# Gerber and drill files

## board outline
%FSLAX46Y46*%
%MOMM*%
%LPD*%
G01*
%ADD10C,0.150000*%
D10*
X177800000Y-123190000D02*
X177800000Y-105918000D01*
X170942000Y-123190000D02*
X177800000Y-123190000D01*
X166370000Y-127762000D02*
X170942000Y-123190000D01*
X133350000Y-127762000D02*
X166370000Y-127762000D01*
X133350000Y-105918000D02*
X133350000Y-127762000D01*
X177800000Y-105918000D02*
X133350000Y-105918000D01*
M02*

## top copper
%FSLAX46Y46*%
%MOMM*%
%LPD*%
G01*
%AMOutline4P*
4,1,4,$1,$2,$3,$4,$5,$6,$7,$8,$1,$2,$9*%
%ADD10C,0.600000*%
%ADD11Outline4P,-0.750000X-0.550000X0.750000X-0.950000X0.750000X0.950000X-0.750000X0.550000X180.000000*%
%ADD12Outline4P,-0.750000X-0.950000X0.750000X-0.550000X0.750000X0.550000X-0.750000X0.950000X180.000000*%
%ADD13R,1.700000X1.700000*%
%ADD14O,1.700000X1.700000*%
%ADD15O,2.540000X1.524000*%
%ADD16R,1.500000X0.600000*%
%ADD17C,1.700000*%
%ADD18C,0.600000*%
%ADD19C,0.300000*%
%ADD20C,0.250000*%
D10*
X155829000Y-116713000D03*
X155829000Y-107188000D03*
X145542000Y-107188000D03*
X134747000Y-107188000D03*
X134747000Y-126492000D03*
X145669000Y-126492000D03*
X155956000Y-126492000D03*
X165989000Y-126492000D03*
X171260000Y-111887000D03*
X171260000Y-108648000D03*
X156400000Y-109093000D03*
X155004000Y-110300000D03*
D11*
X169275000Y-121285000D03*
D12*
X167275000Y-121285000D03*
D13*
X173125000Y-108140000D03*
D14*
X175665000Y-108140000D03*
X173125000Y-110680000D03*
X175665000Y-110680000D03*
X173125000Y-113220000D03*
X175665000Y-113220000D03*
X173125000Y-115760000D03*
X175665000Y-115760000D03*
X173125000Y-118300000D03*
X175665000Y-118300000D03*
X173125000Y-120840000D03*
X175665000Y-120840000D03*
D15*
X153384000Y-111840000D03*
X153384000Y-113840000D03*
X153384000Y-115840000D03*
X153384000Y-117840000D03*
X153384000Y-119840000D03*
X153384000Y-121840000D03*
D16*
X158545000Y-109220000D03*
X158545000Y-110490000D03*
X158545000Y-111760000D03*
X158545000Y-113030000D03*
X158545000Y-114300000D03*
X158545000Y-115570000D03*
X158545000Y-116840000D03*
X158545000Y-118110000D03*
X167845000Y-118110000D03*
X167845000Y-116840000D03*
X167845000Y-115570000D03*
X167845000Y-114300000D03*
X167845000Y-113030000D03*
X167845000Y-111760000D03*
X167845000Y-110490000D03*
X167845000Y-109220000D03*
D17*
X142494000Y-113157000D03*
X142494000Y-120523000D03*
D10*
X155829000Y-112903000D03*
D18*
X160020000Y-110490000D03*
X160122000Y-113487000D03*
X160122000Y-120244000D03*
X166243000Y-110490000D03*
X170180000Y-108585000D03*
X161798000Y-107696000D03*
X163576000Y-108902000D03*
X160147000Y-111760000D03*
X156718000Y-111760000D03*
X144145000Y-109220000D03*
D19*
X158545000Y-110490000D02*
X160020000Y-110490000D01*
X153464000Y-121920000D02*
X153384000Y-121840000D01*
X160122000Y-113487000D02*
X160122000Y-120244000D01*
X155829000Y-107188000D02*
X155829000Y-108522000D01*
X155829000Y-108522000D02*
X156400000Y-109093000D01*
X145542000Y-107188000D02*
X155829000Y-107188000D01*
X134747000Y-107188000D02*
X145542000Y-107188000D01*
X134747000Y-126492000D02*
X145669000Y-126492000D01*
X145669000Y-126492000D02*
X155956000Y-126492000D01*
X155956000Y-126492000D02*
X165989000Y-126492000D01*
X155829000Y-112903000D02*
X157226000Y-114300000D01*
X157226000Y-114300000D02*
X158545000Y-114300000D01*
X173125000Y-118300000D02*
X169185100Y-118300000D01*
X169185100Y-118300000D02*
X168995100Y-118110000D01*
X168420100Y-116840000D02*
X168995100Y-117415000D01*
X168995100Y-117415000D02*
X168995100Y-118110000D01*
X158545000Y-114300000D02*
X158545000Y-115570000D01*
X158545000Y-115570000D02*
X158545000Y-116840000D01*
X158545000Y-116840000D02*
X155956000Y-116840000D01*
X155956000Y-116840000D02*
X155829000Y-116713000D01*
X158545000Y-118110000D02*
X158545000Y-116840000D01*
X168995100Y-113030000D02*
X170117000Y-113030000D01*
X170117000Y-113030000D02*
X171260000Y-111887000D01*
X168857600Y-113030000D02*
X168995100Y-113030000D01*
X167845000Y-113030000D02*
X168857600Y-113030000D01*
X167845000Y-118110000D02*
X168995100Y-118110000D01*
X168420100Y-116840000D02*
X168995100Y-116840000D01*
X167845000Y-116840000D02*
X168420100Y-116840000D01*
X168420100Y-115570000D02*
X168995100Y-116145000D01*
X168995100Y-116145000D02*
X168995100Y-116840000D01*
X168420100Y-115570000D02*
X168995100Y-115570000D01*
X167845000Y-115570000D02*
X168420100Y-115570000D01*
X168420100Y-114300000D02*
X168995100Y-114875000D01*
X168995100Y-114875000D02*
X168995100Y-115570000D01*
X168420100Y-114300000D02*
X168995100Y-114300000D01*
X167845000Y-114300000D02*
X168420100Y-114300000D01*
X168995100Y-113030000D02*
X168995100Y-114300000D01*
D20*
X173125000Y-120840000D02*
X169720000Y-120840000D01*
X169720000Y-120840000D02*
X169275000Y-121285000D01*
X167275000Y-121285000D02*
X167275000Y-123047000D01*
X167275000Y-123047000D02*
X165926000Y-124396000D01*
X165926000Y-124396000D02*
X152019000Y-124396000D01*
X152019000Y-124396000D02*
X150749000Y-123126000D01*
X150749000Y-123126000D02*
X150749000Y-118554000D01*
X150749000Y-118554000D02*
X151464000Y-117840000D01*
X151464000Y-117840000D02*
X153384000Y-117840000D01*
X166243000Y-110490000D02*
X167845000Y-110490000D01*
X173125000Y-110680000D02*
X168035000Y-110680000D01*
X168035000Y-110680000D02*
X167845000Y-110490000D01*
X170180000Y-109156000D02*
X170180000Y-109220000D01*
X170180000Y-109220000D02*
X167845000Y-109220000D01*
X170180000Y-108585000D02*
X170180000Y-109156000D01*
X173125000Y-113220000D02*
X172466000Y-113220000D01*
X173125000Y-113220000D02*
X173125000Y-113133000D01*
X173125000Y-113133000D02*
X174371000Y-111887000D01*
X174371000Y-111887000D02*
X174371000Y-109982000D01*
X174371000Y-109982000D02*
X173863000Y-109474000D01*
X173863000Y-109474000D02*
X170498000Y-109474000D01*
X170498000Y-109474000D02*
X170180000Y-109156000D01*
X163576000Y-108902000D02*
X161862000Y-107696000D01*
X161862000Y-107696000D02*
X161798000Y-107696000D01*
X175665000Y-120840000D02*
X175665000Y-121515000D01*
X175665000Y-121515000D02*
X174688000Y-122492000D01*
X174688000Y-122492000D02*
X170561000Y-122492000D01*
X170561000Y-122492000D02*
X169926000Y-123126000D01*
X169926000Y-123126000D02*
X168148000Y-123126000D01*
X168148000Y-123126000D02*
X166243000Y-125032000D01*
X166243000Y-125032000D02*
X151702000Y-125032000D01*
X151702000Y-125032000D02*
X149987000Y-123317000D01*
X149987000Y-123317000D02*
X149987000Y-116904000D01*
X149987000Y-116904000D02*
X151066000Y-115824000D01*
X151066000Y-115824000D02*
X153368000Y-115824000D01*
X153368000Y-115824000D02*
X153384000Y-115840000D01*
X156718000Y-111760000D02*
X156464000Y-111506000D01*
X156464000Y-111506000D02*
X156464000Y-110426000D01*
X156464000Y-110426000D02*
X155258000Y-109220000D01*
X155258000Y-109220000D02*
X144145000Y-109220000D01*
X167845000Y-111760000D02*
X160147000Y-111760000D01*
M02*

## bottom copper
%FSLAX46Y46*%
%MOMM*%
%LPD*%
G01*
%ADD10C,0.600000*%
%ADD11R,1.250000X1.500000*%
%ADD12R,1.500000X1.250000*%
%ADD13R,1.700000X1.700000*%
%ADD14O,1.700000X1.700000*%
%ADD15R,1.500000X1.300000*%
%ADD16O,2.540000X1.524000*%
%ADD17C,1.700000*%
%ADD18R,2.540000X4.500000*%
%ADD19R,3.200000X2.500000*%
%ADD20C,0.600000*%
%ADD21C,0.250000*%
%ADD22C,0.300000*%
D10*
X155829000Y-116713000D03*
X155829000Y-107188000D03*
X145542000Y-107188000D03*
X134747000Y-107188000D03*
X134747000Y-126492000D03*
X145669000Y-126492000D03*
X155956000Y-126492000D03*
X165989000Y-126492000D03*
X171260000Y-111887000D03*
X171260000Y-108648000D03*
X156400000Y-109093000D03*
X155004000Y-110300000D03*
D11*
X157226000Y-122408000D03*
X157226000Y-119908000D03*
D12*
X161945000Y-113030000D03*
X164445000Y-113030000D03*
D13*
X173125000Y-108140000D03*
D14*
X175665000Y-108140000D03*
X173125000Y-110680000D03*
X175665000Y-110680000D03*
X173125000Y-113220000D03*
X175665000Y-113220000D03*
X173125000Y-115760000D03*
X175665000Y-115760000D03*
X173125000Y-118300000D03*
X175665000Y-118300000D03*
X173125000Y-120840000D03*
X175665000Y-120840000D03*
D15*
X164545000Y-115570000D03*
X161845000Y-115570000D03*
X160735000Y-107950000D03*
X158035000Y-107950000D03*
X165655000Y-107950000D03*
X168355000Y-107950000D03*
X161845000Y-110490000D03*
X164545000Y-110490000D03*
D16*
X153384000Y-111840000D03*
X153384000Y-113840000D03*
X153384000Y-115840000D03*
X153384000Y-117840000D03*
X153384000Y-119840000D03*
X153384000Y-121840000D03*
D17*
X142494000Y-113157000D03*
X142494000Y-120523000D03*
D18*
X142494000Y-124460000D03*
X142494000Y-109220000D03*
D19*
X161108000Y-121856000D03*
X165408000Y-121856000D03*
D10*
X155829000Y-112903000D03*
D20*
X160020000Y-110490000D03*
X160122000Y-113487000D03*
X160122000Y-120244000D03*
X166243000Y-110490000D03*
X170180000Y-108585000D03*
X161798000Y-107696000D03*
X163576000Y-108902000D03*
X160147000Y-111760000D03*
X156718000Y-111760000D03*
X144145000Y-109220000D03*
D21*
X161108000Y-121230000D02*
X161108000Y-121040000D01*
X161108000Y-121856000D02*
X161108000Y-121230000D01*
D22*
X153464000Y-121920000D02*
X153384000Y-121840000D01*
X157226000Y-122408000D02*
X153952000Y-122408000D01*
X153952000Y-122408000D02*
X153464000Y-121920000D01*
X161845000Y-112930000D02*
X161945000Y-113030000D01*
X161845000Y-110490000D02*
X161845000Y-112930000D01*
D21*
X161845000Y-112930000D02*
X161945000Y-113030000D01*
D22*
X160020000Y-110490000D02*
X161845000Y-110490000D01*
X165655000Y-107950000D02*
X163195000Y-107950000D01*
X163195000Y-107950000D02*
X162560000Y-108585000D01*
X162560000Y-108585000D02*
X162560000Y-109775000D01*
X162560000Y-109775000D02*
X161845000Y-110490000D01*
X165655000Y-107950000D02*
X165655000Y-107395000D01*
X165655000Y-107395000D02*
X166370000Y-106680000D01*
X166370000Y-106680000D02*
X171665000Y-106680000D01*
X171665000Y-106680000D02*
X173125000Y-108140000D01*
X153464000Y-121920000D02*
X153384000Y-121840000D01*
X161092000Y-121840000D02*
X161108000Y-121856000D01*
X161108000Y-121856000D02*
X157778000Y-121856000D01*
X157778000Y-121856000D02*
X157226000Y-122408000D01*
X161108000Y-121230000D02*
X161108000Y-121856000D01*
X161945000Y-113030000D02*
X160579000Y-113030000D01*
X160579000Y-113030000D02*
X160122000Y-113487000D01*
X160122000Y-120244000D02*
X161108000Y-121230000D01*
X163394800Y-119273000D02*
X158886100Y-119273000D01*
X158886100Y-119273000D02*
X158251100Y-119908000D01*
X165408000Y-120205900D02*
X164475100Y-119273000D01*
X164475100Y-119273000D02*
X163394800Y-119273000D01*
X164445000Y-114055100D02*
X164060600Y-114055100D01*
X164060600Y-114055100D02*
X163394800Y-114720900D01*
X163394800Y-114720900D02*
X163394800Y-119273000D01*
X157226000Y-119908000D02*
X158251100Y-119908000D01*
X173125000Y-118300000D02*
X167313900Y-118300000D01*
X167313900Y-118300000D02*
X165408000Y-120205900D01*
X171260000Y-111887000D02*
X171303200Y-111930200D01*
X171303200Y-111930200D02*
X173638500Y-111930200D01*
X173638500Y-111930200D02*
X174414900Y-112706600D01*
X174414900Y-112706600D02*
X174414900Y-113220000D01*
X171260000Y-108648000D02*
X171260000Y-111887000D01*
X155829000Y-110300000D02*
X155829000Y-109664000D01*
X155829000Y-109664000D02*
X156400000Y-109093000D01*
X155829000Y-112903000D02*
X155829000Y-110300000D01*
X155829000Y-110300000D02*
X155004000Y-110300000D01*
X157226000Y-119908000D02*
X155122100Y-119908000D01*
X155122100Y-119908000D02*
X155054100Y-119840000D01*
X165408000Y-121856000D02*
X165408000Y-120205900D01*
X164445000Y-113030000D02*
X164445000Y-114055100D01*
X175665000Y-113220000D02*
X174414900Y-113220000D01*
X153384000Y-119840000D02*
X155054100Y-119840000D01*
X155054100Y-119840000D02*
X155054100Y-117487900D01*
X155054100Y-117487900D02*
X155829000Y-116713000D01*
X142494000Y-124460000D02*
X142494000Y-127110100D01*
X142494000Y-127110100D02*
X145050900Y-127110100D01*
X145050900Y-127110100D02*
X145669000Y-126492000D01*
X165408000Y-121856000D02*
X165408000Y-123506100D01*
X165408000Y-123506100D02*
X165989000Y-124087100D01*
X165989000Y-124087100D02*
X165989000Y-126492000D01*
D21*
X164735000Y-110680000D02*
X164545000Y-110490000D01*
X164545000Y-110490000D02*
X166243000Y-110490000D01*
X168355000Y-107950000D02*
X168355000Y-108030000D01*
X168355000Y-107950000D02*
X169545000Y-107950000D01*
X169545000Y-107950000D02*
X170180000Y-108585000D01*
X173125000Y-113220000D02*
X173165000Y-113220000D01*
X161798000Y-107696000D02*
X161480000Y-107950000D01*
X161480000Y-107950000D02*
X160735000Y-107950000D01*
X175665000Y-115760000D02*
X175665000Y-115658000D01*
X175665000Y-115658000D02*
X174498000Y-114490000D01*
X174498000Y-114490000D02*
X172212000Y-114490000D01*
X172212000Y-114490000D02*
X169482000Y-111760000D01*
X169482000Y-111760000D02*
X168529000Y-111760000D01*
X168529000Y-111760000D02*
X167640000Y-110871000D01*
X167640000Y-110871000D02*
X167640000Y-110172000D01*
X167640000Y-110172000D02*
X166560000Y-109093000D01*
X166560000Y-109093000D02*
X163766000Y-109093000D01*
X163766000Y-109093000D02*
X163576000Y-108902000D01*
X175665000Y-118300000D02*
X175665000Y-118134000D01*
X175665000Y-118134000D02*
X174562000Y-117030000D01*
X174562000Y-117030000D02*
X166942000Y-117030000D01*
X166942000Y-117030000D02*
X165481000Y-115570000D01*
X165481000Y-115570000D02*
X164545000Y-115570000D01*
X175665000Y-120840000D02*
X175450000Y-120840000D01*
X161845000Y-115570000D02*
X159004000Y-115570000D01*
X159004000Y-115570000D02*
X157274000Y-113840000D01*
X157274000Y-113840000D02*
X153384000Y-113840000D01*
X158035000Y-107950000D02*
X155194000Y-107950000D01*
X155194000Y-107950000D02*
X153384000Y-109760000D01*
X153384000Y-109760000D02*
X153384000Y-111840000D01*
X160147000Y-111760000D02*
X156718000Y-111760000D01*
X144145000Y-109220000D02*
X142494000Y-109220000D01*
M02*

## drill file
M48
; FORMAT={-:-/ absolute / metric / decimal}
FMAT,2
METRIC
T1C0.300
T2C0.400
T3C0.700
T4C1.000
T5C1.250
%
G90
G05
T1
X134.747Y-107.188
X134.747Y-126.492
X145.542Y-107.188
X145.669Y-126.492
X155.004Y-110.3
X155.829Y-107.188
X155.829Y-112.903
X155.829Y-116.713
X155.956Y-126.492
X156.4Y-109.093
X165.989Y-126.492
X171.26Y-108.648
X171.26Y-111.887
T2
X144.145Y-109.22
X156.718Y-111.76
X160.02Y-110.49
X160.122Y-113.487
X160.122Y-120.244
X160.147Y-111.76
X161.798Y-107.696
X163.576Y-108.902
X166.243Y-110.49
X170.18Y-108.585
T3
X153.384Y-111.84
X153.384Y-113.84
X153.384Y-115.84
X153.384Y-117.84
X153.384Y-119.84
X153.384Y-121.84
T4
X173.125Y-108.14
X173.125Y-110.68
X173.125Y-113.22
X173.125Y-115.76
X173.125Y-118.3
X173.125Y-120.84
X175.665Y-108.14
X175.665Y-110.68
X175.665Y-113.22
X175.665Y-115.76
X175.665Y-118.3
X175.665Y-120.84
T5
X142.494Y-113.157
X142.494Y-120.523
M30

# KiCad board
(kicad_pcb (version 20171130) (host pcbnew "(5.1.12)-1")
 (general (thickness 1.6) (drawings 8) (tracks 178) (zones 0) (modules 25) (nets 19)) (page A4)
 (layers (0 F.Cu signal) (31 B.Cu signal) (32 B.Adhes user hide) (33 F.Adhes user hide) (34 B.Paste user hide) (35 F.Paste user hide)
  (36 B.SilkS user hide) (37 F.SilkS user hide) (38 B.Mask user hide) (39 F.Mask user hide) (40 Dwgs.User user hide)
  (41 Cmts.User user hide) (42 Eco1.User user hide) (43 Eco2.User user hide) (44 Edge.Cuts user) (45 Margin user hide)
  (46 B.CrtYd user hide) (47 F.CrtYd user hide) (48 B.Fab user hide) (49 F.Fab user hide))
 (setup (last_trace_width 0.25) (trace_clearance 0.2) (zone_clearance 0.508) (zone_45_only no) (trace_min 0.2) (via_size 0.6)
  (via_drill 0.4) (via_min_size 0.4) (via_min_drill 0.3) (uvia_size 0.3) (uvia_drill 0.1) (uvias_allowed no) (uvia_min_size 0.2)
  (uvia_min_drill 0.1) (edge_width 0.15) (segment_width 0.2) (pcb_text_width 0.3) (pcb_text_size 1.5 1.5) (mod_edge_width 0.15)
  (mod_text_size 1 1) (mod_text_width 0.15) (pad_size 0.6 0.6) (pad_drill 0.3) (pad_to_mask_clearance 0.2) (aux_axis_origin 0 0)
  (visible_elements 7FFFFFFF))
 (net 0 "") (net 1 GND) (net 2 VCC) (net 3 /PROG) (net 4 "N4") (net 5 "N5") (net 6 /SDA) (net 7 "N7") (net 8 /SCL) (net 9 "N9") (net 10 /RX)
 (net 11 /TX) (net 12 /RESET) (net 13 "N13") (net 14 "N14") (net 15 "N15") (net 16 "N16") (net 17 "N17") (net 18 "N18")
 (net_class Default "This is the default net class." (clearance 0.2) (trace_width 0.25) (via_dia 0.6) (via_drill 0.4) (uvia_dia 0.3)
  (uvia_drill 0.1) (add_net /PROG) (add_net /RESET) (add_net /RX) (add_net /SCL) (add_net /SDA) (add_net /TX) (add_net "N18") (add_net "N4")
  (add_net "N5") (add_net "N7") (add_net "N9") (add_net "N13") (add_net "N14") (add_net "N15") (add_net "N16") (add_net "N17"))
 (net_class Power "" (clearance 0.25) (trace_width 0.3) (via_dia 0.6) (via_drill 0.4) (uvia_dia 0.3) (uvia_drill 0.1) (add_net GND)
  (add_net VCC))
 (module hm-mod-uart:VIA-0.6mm (layer F.Cu) (at 155.829 116.713)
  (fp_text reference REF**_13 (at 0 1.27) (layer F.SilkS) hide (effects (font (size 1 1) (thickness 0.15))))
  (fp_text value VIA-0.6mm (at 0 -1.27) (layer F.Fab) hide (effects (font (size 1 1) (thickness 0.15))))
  (pad 1 thru_hole circle (at 0 0) (size 0.6 0.6) (drill 0.3) (layers *.Cu) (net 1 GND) (zone_connect 2)))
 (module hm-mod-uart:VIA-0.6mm (layer F.Cu) (at 155.829 107.188)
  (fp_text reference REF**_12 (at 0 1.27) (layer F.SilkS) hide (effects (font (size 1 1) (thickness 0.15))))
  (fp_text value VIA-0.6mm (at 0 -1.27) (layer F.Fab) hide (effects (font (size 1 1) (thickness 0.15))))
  (pad 1 thru_hole circle (at 0 0) (size 0.6 0.6) (drill 0.3) (layers *.Cu) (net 1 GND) (zone_connect 2)))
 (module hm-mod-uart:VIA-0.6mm (layer F.Cu) (at 145.542 107.188)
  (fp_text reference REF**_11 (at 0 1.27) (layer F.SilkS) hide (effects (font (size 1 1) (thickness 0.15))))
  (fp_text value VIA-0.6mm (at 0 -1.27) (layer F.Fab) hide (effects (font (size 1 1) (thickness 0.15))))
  (pad 1 thru_hole circle (at 0 0) (size 0.6 0.6) (drill 0.3) (layers *.Cu) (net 1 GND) (zone_connect 2)))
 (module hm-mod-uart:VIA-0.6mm (layer F.Cu) (at 134.747 107.188)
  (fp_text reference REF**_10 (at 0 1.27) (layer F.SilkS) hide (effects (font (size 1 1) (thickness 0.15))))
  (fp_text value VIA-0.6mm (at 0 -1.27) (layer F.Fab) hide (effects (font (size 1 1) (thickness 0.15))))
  (pad 1 thru_hole circle (at 0 0) (size 0.6 0.6) (drill 0.3) (layers *.Cu) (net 1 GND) (zone_connect 2)))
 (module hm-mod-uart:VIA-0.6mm (layer F.Cu) (at 134.747 126.492)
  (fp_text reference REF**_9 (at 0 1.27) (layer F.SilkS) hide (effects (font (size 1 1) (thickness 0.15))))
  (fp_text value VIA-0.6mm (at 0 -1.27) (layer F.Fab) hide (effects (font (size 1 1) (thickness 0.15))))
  (pad 1 thru_hole circle (at 0 0) (size 0.6 0.6) (drill 0.3) (layers *.Cu) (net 1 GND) (zone_connect 2)))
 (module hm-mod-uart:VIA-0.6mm (layer F.Cu) (at 145.669 126.492)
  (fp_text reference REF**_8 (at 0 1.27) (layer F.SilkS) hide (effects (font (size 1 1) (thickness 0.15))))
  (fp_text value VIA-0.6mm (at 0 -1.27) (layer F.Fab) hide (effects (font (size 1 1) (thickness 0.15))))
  (pad 1 thru_hole circle (at 0 0) (size 0.6 0.6) (drill 0.3) (layers *.Cu) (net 1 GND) (zone_connect 2)))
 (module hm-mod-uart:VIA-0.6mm (layer F.Cu) (at 155.956 126.492)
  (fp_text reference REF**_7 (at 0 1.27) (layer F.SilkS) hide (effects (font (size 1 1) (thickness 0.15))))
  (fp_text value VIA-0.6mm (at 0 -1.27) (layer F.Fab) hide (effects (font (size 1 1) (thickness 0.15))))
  (pad 1 thru_hole circle (at 0 0) (size 0.6 0.6) (drill 0.3) (layers *.Cu) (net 1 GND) (zone_connect 2)))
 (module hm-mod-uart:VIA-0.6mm (layer F.Cu) (at 165.989 126.492)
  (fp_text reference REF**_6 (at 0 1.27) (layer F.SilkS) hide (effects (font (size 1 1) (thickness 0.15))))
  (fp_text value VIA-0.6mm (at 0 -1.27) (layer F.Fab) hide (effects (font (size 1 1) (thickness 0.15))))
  (pad 1 thru_hole circle (at 0 0) (size 0.6 0.6) (drill 0.3) (layers *.Cu) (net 1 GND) (zone_connect 2)))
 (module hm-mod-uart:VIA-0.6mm (layer F.Cu) (at 171.26 111.887)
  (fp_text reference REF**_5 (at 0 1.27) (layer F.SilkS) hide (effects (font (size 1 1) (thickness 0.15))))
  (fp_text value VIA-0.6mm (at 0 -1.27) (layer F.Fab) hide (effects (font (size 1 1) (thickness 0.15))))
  (pad 1 thru_hole circle (at 0 0) (size 0.6 0.6) (drill 0.3) (layers *.Cu) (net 1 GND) (zone_connect 2)))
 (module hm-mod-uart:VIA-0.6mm (layer F.Cu) (at 171.26 108.648)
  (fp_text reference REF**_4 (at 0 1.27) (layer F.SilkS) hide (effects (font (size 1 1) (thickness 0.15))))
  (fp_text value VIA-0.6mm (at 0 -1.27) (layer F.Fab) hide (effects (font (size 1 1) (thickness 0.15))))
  (pad 1 thru_hole circle (at 0 0) (size 0.6 0.6) (drill 0.3) (layers *.Cu) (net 1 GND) (zone_connect 2)))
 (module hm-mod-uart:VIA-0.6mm (layer F.Cu) (at 156.4 109.093)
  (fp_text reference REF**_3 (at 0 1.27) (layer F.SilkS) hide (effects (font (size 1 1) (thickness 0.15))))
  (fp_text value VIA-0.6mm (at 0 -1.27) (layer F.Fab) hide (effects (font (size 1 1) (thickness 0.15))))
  (pad 1 thru_hole circle (at 0 0) (size 0.6 0.6) (drill 0.3) (layers *.Cu) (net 1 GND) (zone_connect 2)))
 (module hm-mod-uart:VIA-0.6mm (layer F.Cu) (at 155.004 110.3)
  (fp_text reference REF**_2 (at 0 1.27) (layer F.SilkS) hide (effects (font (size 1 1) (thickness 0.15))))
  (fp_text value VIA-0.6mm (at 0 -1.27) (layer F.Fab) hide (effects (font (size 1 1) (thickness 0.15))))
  (pad 1 thru_hole circle (at 0 0) (size 0.6 0.6) (drill 0.3) (layers *.Cu) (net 1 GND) (zone_connect 2)))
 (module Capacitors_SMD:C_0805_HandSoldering (layer B.Cu) (at 157.226 121.158 90)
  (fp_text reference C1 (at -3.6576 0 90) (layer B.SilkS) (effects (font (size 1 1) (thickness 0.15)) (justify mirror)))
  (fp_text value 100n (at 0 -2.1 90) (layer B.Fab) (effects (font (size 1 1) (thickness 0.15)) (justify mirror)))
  (pad 1 smd rect (at -1.25 0 90) (size 1.5 1.25) (layers B.Cu B.Paste B.Mask) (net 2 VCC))
  (pad 2 smd rect (at 1.25 0 90) (size 1.5 1.25) (layers B.Cu B.Paste B.Mask) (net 1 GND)))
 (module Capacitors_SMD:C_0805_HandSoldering (layer B.Cu) (at 163.195 113.03)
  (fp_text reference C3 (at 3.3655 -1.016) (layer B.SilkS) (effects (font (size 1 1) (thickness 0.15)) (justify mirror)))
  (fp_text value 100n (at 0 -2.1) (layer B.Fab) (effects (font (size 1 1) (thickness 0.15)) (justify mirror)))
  (pad 1 smd rect (at -1.25 0) (size 1.5 1.25) (layers B.Cu B.Paste B.Mask) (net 2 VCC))
  (pad 2 smd rect (at 1.25 0) (size 1.5 1.25) (layers B.Cu B.Paste B.Mask) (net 1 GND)))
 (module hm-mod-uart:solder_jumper (layer F.Cu) (at 168.275 121.285 180)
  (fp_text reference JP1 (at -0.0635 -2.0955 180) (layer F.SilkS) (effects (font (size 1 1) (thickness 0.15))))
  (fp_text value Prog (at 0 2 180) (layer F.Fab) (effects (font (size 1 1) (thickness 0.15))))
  (pad 1 smd trapezoid (at -1 0 180) (size 1.5 1.5) (rect_delta -0.4 0) (layers F.Cu F.Paste F.Mask) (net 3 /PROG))
  (pad 2 smd trapezoid (at 1 0 180) (size 1.5 1.5) (rect_delta 0.4 0) (layers F.Cu F.Paste F.Mask) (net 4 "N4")))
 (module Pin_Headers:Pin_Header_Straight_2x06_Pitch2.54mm (layer F.Cu) (at 173.125 108.14)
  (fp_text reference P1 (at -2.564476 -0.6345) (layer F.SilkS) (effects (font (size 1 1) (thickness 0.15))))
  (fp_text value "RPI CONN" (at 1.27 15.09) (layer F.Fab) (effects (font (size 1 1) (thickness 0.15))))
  (pad 1 thru_hole rect (at 0 0) (size 1.7 1.7) (drill 1) (layers *.Cu *.Mask) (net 2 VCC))
  (pad 2 thru_hole oval (at 2.54 0) (size 1.7 1.7) (drill 1) (layers *.Cu *.Mask) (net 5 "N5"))
  (pad 3 thru_hole oval (at 0 2.54) (size 1.7 1.7) (drill 1) (layers *.Cu *.Mask) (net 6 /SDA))
  (pad 4 thru_hole oval (at 2.54 2.54) (size 1.7 1.7) (drill 1) (layers *.Cu *.Mask) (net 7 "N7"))
  (pad 5 thru_hole oval (at 0 5.08) (size 1.7 1.7) (drill 1) (layers *.Cu *.Mask) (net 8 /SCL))
  (pad 6 thru_hole oval (at 2.54 5.08) (size 1.7 1.7) (drill 1) (layers *.Cu *.Mask) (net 1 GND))
  (pad 7 thru_hole oval (at 0 7.62) (size 1.7 1.7) (drill 1) (layers *.Cu *.Mask) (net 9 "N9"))
  (pad 8 thru_hole oval (at 2.54 7.62) (size 1.7 1.7) (drill 1) (layers *.Cu *.Mask) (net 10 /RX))
  (pad 9 thru_hole oval (at 0 10.16) (size 1.7 1.7) (drill 1) (layers *.Cu *.Mask) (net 1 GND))
  (pad 10 thru_hole oval (at 2.54 10.16) (size 1.7 1.7) (drill 1) (layers *.Cu *.Mask) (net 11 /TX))
  (pad 11 thru_hole oval (at 0 12.7) (size 1.7 1.7) (drill 1) (layers *.Cu *.Mask) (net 3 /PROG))
  (pad 12 thru_hole oval (at 2.54 12.7) (size 1.7 1.7) (drill 1) (layers *.Cu *.Mask) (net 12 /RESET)))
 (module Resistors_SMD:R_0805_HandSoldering (layer B.Cu) (at 163.195 115.57 180)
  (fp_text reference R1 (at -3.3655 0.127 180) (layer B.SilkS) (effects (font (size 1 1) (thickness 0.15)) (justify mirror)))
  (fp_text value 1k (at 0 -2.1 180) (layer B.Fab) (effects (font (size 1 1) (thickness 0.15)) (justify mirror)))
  (pad 1 smd rect (at -1.35 0 180) (size 1.5 1.3) (layers B.Cu B.Paste B.Mask) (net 11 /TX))
  (pad 2 smd rect (at 1.35 0 180) (size 1.5 1.3) (layers B.Cu B.Paste B.Mask) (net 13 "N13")))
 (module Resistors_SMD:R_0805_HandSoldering (layer B.Cu) (at 159.385 107.95 180)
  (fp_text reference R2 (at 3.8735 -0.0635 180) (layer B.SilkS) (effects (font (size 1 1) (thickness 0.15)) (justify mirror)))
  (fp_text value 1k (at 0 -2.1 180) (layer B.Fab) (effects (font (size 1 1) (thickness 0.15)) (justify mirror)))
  (pad 1 smd rect (at -1.35 0 180) (size 1.5 1.3) (layers B.Cu B.Paste B.Mask) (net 10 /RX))
  (pad 2 smd rect (at 1.35 0 180) (size 1.5 1.3) (layers B.Cu B.Paste B.Mask) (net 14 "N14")))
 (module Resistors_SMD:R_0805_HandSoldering (layer B.Cu) (at 167.005 107.95)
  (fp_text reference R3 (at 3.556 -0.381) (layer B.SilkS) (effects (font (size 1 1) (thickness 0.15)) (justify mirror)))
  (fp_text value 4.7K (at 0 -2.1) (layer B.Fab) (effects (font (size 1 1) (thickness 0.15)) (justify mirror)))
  (pad 1 smd rect (at -1.35 0) (size 1.5 1.3) (layers B.Cu B.Paste B.Mask) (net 2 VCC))
  (pad 2 smd rect (at 1.35 0) (size 1.5 1.3) (layers B.Cu B.Paste B.Mask) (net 8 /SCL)))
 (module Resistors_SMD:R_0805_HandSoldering (layer B.Cu) (at 163.195 110.49)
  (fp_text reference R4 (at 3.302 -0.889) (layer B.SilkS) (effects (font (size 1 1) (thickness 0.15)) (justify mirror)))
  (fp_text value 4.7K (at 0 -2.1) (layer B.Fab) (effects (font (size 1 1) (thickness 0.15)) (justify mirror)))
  (pad 1 smd rect (at -1.35 0) (size 1.5 1.3) (layers B.Cu B.Paste B.Mask) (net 2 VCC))
  (pad 2 smd rect (at 1.35 0) (size 1.5 1.3) (layers B.Cu B.Paste B.Mask) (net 6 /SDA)))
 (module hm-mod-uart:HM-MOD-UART (layer F.Cu) (at 151.384 116.84)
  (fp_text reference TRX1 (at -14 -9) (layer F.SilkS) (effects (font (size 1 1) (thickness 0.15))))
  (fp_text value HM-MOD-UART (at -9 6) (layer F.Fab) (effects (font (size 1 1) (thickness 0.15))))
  (pad 6 thru_hole oval (at 2 -5) (size 2.54 1.524) (drill 0.7) (layers *.Cu *.Mask) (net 14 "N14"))
  (pad 5 thru_hole oval (at 2 -3) (size 2.54 1.524) (drill 0.7) (layers *.Cu *.Mask) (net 13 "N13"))
  (pad 4 thru_hole oval (at 2 -1) (size 2.54 1.524) (drill 0.7) (layers *.Cu *.Mask) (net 12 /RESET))
  (pad 3 thru_hole oval (at 2 1) (size 2.54 1.524) (drill 0.7) (layers *.Cu *.Mask) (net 4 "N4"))
  (pad 2 thru_hole oval (at 2 3) (size 2.54 1.524) (drill 0.7) (layers *.Cu *.Mask) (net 1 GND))
  (pad 1 thru_hole oval (at 2 5) (size 2.54 1.524) (drill 0.7) (layers *.Cu *.Mask) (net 2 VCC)))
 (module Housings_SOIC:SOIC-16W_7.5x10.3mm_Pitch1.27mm (layer F.Cu) (at 163.195 113.665)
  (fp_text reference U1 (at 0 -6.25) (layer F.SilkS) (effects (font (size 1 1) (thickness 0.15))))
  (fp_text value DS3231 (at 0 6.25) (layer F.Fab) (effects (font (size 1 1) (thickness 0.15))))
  (pad 1 smd rect (at -4.65 -4.445) (size 1.5 0.6) (layers F.Cu F.Paste F.Mask) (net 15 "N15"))
  (pad 2 smd rect (at -4.65 -3.175) (size 1.5 0.6) (layers F.Cu F.Paste F.Mask) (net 2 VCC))
  (pad 3 smd rect (at -4.65 -1.905) (size 1.5 0.6) (layers F.Cu F.Paste F.Mask) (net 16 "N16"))
  (pad 4 smd rect (at -4.65 -0.635) (size 1.5 0.6) (layers F.Cu F.Paste F.Mask) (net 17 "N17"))
  (pad 5 smd rect (at -4.65 0.635) (size 1.5 0.6) (layers F.Cu F.Paste F.Mask) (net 1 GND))
  (pad 6 smd rect (at -4.65 1.905) (size 1.5 0.6) (layers F.Cu F.Paste F.Mask) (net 1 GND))
  (pad 7 smd rect (at -4.65 3.175) (size 1.5 0.6) (layers F.Cu F.Paste F.Mask) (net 1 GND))
  (pad 8 smd rect (at -4.65 4.445) (size 1.5 0.6) (layers F.Cu F.Paste F.Mask) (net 1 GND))
  (pad 9 smd rect (at 4.65 4.445) (size 1.5 0.6) (layers F.Cu F.Paste F.Mask) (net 1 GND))
  (pad 10 smd rect (at 4.65 3.175) (size 1.5 0.6) (layers F.Cu F.Paste F.Mask) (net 1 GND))
  (pad 11 smd rect (at 4.65 1.905) (size 1.5 0.6) (layers F.Cu F.Paste F.Mask) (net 1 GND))
  (pad 12 smd rect (at 4.65 0.635) (size 1.5 0.6) (layers F.Cu F.Paste F.Mask) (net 1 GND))
  (pad 13 smd rect (at 4.65 -0.635) (size 1.5 0.6) (layers F.Cu F.Paste F.Mask) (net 1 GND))
  (pad 14 smd rect (at 4.65 -1.905) (size 1.5 0.6) (layers F.Cu F.Paste F.Mask) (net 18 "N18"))
  (pad 15 smd rect (at 4.65 -3.175) (size 1.5 0.6) (layers F.Cu F.Paste F.Mask) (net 6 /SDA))
  (pad 16 smd rect (at 4.65 -4.445) (size 1.5 0.6) (layers F.Cu F.Paste F.Mask) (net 8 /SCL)))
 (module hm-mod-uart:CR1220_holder (layer B.Cu) (at 142.494 116.84 90)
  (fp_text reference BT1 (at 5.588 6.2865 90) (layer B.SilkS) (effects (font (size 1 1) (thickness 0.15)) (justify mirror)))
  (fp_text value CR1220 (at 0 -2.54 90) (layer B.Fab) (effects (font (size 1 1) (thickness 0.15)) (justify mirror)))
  (pad "" np_thru_hole circle (at 3.683 0 90) (size 1.7 1.7) (drill 1.25) (layers *.Cu *.Mask))
  (pad "" np_thru_hole circle (at -3.683 0 90) (size 1.7 1.7) (drill 1.25) (layers *.Cu *.Mask))
  (pad 2 smd rect (at -7.62 0 90) (size 4.5 2.54) (layers B.Cu B.Paste B.Mask) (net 1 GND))
  (pad 1 smd rect (at 7.62 0 90) (size 4.5 2.54) (layers B.Cu B.Paste B.Mask) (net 18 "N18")))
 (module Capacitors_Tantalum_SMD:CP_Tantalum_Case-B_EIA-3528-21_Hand (layer B.Cu) (at 163.258 121.856)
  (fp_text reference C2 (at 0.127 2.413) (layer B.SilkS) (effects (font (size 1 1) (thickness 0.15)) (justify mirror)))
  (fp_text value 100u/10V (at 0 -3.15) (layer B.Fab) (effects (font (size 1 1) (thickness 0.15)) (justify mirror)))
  (pad 1 smd rect (at -2.15 0) (size 3.2 2.5) (layers B.Cu B.Paste B.Mask) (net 2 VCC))
  (pad 2 smd rect (at 2.15 0) (size 3.2 2.5) (layers B.Cu B.Paste B.Mask) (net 1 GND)))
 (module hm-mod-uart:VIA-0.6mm (layer F.Cu) (at 155.829 112.903)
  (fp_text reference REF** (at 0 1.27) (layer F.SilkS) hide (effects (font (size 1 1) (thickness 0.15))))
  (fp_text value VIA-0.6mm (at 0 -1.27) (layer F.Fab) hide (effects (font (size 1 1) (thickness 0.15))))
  (pad 1 thru_hole circle (at 0 0) (size 0.6 0.6) (drill 0.3) (layers *.Cu) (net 1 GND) (zone_connect 2)))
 (gr_line (start 177.8 123.19) (end 177.8 105.918) (angle 90) (layer Edge.Cuts) (width 0.15))
 (gr_line (start 170.942 123.19) (end 177.8 123.19) (angle 90) (layer Edge.Cuts) (width 0.15))
 (gr_line (start 166.37 127.762) (end 170.942 123.19) (angle 90) (layer Edge.Cuts) (width 0.15))
 (gr_line (start 133.35 127.762) (end 166.37 127.762) (angle 90) (layer Edge.Cuts) (width 0.15))
 (gr_line (start 133.35 105.918) (end 133.35 127.762) (angle 90) (layer Edge.Cuts) (width 0.15))
 (gr_line (start 177.8 105.918) (end 133.35 105.918) (angle 90) (layer Edge.Cuts) (width 0.15))
 (segment (start 161.108 121.23) (end 161.108 121.04) (width 0.25) (layer B.Cu) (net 2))
 (segment (start 161.108 121.856) (end 161.108 121.23) (width 0.25) (layer B.Cu) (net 2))
 (segment (start 153.464 121.92) (end 153.384 121.84) (width 0.3) (layer B.Cu) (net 2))
 (segment (start 157.226 122.408) (end 153.952 122.408) (width 0.3) (layer B.Cu) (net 2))
 (segment (start 153.952 122.408) (end 153.464 121.92) (width 0.3) (layer B.Cu) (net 2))
 (segment (start 161.845 112.93) (end 161.945 113.03) (width 0.3) (layer B.Cu) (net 2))
 (segment (start 161.845 110.49) (end 161.845 112.93) (width 0.3) (layer B.Cu) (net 2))
 (segment (start 161.845 112.93) (end 161.945 113.03) (width 0.25) (layer B.Cu) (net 2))
 (segment (start 160.02 110.49) (end 161.845 110.49) (width 0.3) (layer B.Cu) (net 2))
 (segment (start 158.545 110.49) (end 160.02 110.49) (width 0.3) (layer F.Cu) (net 2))
 (segment (start 165.655 107.95) (end 163.195 107.95) (width 0.3) (layer B.Cu) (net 2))
 (segment (start 163.195 107.95) (end 162.56 108.585) (width 0.3) (layer B.Cu) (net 2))
 (segment (start 162.56 108.585) (end 162.56 109.775) (width 0.3) (layer B.Cu) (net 2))
 (segment (start 162.56 109.775) (end 161.845 110.49) (width 0.3) (layer B.Cu) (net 2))
 (segment (start 165.655 107.95) (end 165.655 107.395) (width 0.3) (layer B.Cu) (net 2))
 (segment (start 165.655 107.395) (end 166.37 106.68) (width 0.3) (layer B.Cu) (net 2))
 (segment (start 166.37 106.68) (end 171.665 106.68) (width 0.3) (layer B.Cu) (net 2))
 (segment (start 171.665 106.68) (end 173.125 108.14) (width 0.3) (layer B.Cu) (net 2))
 (segment (start 153.464 121.92) (end 153.384 121.84) (width 0.3) (layer F.Cu) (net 2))
 (segment (start 153.464 121.92) (end 153.384 121.84) (width 0.3) (layer B.Cu) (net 2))
 (segment (start 161.092 121.84) (end 161.108 121.856) (width 0.3) (layer B.Cu) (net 2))
 (segment (start 161.108 121.856) (end 157.778 121.856) (width 0.3) (layer B.Cu) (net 2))
 (segment (start 157.778 121.856) (end 157.226 122.408) (width 0.3) (layer B.Cu) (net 2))
 (segment (start 161.108 121.23) (end 161.108 121.856) (width 0.3) (layer B.Cu) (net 2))
 (segment (start 161.945 113.03) (end 160.579 113.03) (width 0.3) (layer B.Cu) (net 2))
 (segment (start 160.579 113.03) (end 160.122 113.487) (width 0.3) (layer B.Cu) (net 2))
 (segment (start 160.122 113.487) (end 160.122 120.244) (width 0.3) (layer F.Cu) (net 2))
 (segment (start 160.122 120.244) (end 161.108 121.23) (width 0.3) (layer B.Cu) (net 2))
 (via (at 160.02 110.49) (size 0.6) (layers F.Cu B.Cu) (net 2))
 (via (at 160.122 113.487) (size 0.6) (layers F.Cu B.Cu) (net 2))
 (via (at 160.122 120.244) (size 0.6) (layers F.Cu B.Cu) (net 2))
 (segment (start 155.829 107.188) (end 155.829 108.522) (width 0.3) (layer F.Cu) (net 1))
 (segment (start 155.829 108.522) (end 156.4 109.093) (width 0.3) (layer F.Cu) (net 1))
 (segment (start 145.542 107.188) (end 155.829 107.188) (width 0.3) (layer F.Cu) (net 1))
 (segment (start 134.747 107.188) (end 145.542 107.188) (width 0.3) (layer F.Cu) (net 1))
 (segment (start 134.747 126.492) (end 145.669 126.492) (width 0.3) (layer F.Cu) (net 1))
 (segment (start 145.669 126.492) (end 155.956 126.492) (width 0.3) (layer F.Cu) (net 1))
 (segment (start 155.956 126.492) (end 165.989 126.492) (width 0.3) (layer F.Cu) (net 1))
 (segment (start 163.3948 119.273) (end 158.8861 119.273) (width 0.3) (layer B.Cu) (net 1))
 (segment (start 158.8861 119.273) (end 158.2511 119.908) (width 0.3) (layer B.Cu) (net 1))
 (segment (start 165.408 120.2059) (end 164.4751 119.273) (width 0.3) (layer B.Cu) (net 1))
 (segment (start 164.4751 119.273) (end 163.3948 119.273) (width 0.3) (layer B.Cu) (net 1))
 (segment (start 164.445 114.0551) (end 164.0606 114.0551) (width 0.3) (layer B.Cu) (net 1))
 (segment (start 164.0606 114.0551) (end 163.3948 114.7209) (width 0.3) (layer B.Cu) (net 1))
 (segment (start 163.3948 114.7209) (end 163.3948 119.273) (width 0.3) (layer B.Cu) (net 1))
 (segment (start 157.226 119.908) (end 158.2511 119.908) (width 0.3) (layer B.Cu) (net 1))
 (segment (start 173.125 118.3) (end 167.3139 118.3) (width 0.3) (layer B.Cu) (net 1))
 (segment (start 167.3139 118.3) (end 165.408 120.2059) (width 0.3) (layer B.Cu) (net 1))
 (segment (start 171.26 111.887) (end 171.3032 111.9302) (width 0.3) (layer B.Cu) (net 1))
 (segment (start 171.3032 111.9302) (end 173.6385 111.9302) (width 0.3) (layer B.Cu) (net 1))
 (segment (start 173.6385 111.9302) (end 174.4149 112.7066) (width 0.3) (layer B.Cu) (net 1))
 (segment (start 174.4149 112.7066) (end 174.4149 113.22) (width 0.3) (layer B.Cu) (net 1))
 (segment (start 171.26 108.648) (end 171.26 111.887) (width 0.3) (layer B.Cu) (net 1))
 (segment (start 155.829 112.903) (end 157.226 114.3) (width 0.3) (layer F.Cu) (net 1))
 (segment (start 157.226 114.3) (end 158.545 114.3) (width 0.3) (layer F.Cu) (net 1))
 (segment (start 155.829 110.3) (end 155.829 109.664) (width 0.3) (layer B.Cu) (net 1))
 (segment (start 155.829 109.664) (end 156.4 109.093) (width 0.3) (layer B.Cu) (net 1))
 (segment (start 155.829 112.903) (end 155.829 110.3) (width 0.3) (layer B.Cu) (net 1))
 (segment (start 155.829 110.3) (end 155.004 110.3) (width 0.3) (layer B.Cu) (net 1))
 (segment (start 157.226 119.908) (end 155.1221 119.908) (width 0.3) (layer B.Cu) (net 1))
 (segment (start 155.1221 119.908) (end 155.0541 119.84) (width 0.3) (layer B.Cu) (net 1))
 (segment (start 165.408 121.856) (end 165.408 120.2059) (width 0.3) (layer B.Cu) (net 1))
 (segment (start 164.445 113.03) (end 164.445 114.0551) (width 0.3) (layer B.Cu) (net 1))
 (segment (start 175.665 113.22) (end 174.4149 113.22) (width 0.3) (layer B.Cu) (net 1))
 (segment (start 173.125 118.3) (end 169.1851 118.3) (width 0.3) (layer F.Cu) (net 1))
 (segment (start 169.1851 118.3) (end 168.9951 118.11) (width 0.3) (layer F.Cu) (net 1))
 (segment (start 168.4201 116.84) (end 168.9951 117.415) (width 0.3) (layer F.Cu) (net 1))
 (segment (start 168.9951 117.415) (end 168.9951 118.11) (width 0.3) (layer F.Cu) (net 1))
 (segment (start 153.384 119.84) (end 155.0541 119.84) (width 0.3) (layer B.Cu) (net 1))
 (segment (start 155.0541 119.84) (end 155.0541 117.4879) (width 0.3) (layer B.Cu) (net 1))
 (segment (start 155.0541 117.4879) (end 155.829 116.713) (width 0.3) (layer B.Cu) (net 1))
 (segment (start 158.545 114.3) (end 158.545 115.57) (width 0.3) (layer F.Cu) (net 1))
 (segment (start 158.545 115.57) (end 158.545 116.84) (width 0.3) (layer F.Cu) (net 1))
 (segment (start 158.545 116.84) (end 155.956 116.84) (width 0.3) (layer F.Cu) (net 1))
 (segment (start 155.956 116.84) (end 155.829 116.713) (width 0.3) (layer F.Cu) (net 1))
 (segment (start 158.545 118.11) (end 158.545 116.84) (width 0.3) (layer F.Cu) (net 1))
 (segment (start 168.9951 113.03) (end 170.117 113.03) (width 0.3) (layer F.Cu) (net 1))
 (segment (start 170.117 113.03) (end 171.26 111.887) (width 0.3) (layer F.Cu) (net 1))
 (segment (start 168.8576 113.03) (end 168.9951 113.03) (width 0.3) (layer F.Cu) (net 1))
 (segment (start 167.845 113.03) (end 168.8576 113.03) (width 0.3) (layer F.Cu) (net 1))
 (segment (start 167.845 118.11) (end 168.9951 118.11) (width 0.3) (layer F.Cu) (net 1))
 (segment (start 168.4201 116.84) (end 168.9951 116.84) (width 0.3) (layer F.Cu) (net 1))
 (segment (start 167.845 116.84) (end 168.4201 116.84) (width 0.3) (layer F.Cu) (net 1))
 (segment (start 168.4201 115.57) (end 168.9951 116.145) (width 0.3) (layer F.Cu) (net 1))
 (segment (start 168.9951 116.145) (end 168.9951 116.84) (width 0.3) (layer F.Cu) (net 1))
 (segment (start 168.4201 115.57) (end 168.9951 115.57) (width 0.3) (layer F.Cu) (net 1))
 (segment (start 167.845 115.57) (end 168.4201 115.57) (width 0.3) (layer F.Cu) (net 1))
 (segment (start 168.4201 114.3) (end 168.9951 114.875) (width 0.3) (layer F.Cu) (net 1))
 (segment (start 168.9951 114.875) (end 168.9951 115.57) (width 0.3) (layer F.Cu) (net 1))
 (segment (start 168.4201 114.3) (end 168.9951 114.3) (width 0.3) (layer F.Cu) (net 1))
 (segment (start 167.845 114.3) (end 168.4201 114.3) (width 0.3) (layer F.Cu) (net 1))
 (segment (start 168.9951 113.03) (end 168.9951 114.3) (width 0.3) (layer F.Cu) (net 1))
 (segment (start 142.494 124.46) (end 142.494 127.1101) (width 0.3) (layer B.Cu) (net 1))
 (segment (start 142.494 127.1101) (end 145.0509 127.1101) (width 0.3) (layer B.Cu) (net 1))
 (segment (start 145.0509 127.1101) (end 145.669 126.492) (width 0.3) (layer B.Cu) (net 1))
 (segment (start 165.408 121.856) (end 165.408 123.5061) (width 0.3) (layer B.Cu) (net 1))
 (segment (start 165.408 123.5061) (end 165.989 124.0871) (width 0.3) (layer B.Cu) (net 1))
 (segment (start 165.989 124.0871) (end 165.989 126.492) (width 0.3) (layer B.Cu) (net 1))
 (segment (start 173.125 120.84) (end 169.72 120.84) (width 0.25) (layer F.Cu) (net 3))
 (segment (start 169.72 120.84) (end 169.275 121.285) (width 0.25) (layer F.Cu) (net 3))
 (segment (start 167.275 121.285) (end 167.275 123.047) (width 0.25) (layer F.Cu) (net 4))
 (segment (start 167.275 123.047) (end 165.926 124.396) (width 0.25) (layer F.Cu) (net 4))
 (segment (start 165.926 124.396) (end 152.019 124.396) (width 0.25) (layer F.Cu) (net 4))
 (segment (start 152.019 124.396) (end 150.749 123.126) (width 0.25) (layer F.Cu) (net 4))
 (segment (start 150.749 123.126) (end 150.749 118.554) (width 0.25) (layer F.Cu) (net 4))
 (segment (start 150.749 118.554) (end 151.464 117.84) (width 0.25) (layer F.Cu) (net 4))
 (segment (start 151.464 117.84) (end 153.384 117.84) (width 0.25) (layer F.Cu) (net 4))
 (segment (start 164.735 110.68) (end 164.545 110.49) (width 0.25) (layer B.Cu) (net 6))
 (segment (start 166.243 110.49) (end 167.845 110.49) (width 0.25) (layer F.Cu) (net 6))
 (segment (start 164.545 110.49) (end 166.243 110.49) (width 0.25) (layer B.Cu) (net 6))
 (segment (start 173.125 110.68) (end 168.035 110.68) (width 0.25) (layer F.Cu) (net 6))
 (segment (start 168.035 110.68) (end 167.845 110.49) (width 0.25) (layer F.Cu) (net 6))
 (via (at 166.243 110.49) (size 0.6) (layers F.Cu B.Cu) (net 6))
 (segment (start 170.18 109.156) (end 170.18 109.22) (width 0.25) (layer F.Cu) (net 8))
 (segment (start 170.18 109.22) (end 167.845 109.22) (width 0.25) (layer F.Cu) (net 8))
 (segment (start 170.18 108.585) (end 170.18 109.156) (width 0.25) (layer F.Cu) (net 8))
 (segment (start 168.355 107.95) (end 168.355 108.03) (width 0.25) (layer B.Cu) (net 8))
 (segment (start 168.355 107.95) (end 169.545 107.95) (width 0.25) (layer B.Cu) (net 8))
 (segment (start 169.545 107.95) (end 170.18 108.585) (width 0.25) (layer B.Cu) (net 8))
 (segment (start 173.125 113.22) (end 172.466 113.22) (width 0.25) (layer F.Cu) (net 8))
 (segment (start 173.125 113.22) (end 173.165 113.22) (width 0.25) (layer B.Cu) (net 8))
 (segment (start 173.125 113.22) (end 173.125 113.133) (width 0.25) (layer F.Cu) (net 8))
 (segment (start 173.125 113.133) (end 174.371 111.887) (width 0.25) (layer F.Cu) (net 8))
 (segment (start 174.371 111.887) (end 174.371 109.982) (width 0.25) (layer F.Cu) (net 8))
 (segment (start 174.371 109.982) (end 173.863 109.474) (width 0.25) (layer F.Cu) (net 8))
 (segment (start 173.863 109.474) (end 170.498 109.474) (width 0.25) (layer F.Cu) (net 8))
 (segment (start 170.498 109.474) (end 170.18 109.156) (width 0.25) (layer F.Cu) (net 8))
 (via (at 170.18 108.585) (size 0.6) (layers F.Cu B.Cu) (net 8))
 (segment (start 161.798 107.696) (end 161.48 107.95) (width 0.25) (layer B.Cu) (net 10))
 (segment (start 161.48 107.95) (end 160.735 107.95) (width 0.25) (layer B.Cu) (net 10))
 (segment (start 163.576 108.902) (end 161.862 107.696) (width 0.25) (layer F.Cu) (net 10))
 (segment (start 161.862 107.696) (end 161.798 107.696) (width 0.25) (layer F.Cu) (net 10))
 (segment (start 175.665 115.76) (end 175.665 115.658) (width 0.25) (layer B.Cu) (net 10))
 (segment (start 175.665 115.658) (end 174.498 114.49) (width 0.25) (layer B.Cu) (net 10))
 (segment (start 174.498 114.49) (end 172.212 114.49) (width 0.25) (layer B.Cu) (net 10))
 (segment (start 172.212 114.49) (end 169.482 111.76) (width 0.25) (layer B.Cu) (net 10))
 (segment (start 169.482 111.76) (end 168.529 111.76) (width 0.25) (layer B.Cu) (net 10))
 (segment (start 168.529 111.76) (end 167.64 110.871) (width 0.25) (layer B.Cu) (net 10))
 (segment (start 167.64 110.871) (end 167.64 110.172) (width 0.25) (layer B.Cu) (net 10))
 (segment (start 167.64 110.172) (end 166.56 109.093) (width 0.25) (layer B.Cu) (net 10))
 (segment (start 166.56 109.093) (end 163.766 109.093) (width 0.25) (layer B.Cu) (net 10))
 (segment (start 163.766 109.093) (end 163.576 108.902) (width 0.25) (layer B.Cu) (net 10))
 (via (at 161.798 107.696) (size 0.6) (layers F.Cu B.Cu) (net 10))
 (via (at 163.576 108.902) (size 0.6) (layers F.Cu B.Cu) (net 10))
 (segment (start 175.665 118.3) (end 175.665 118.134) (width 0.25) (layer B.Cu) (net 11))
 (segment (start 175.665 118.134) (end 174.562 117.03) (width 0.25) (layer B.Cu) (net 11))
 (segment (start 174.562 117.03) (end 166.942 117.03) (width 0.25) (layer B.Cu) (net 11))
 (segment (start 166.942 117.03) (end 165.481 115.57) (width 0.25) (layer B.Cu) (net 11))
 (segment (start 165.481 115.57) (end 164.545 115.57) (width 0.25) (layer B.Cu) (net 11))
 (segment (start 175.665 120.84) (end 175.45 120.84) (width 0.25) (layer B.Cu) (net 12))
 (segment (start 175.665 120.84) (end 175.665 121.515) (width 0.25) (layer F.Cu) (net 12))
 (segment (start 175.665 121.515) (end 174.688 122.492) (width 0.25) (layer F.Cu) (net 12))
 (segment (start 174.688 122.492) (end 170.561 122.492) (width 0.25) (layer F.Cu) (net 12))
 (segment (start 170.561 122.492) (end 169.926 123.126) (width 0.25) (layer F.Cu) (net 12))
 (segment (start 169.926 123.126) (end 168.148 123.126) (width 0.25) (layer F.Cu) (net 12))
 (segment (start 168.148 123.126) (end 166.243 125.032) (width 0.25) (layer F.Cu) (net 12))
 (segment (start 166.243 125.032) (end 151.702 125.032) (width 0.25) (layer F.Cu) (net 12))
 (segment (start 151.702 125.032) (end 149.987 123.317) (width 0.25) (layer F.Cu) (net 12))
 (segment (start 149.987 123.317) (end 149.987 116.904) (width 0.25) (layer F.Cu) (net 12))
 (segment (start 149.987 116.904) (end 151.066 115.824) (width 0.25) (layer F.Cu) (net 12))
 (segment (start 151.066 115.824) (end 153.368 115.824) (width 0.25) (layer F.Cu) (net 12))
 (segment (start 153.368 115.824) (end 153.384 115.84) (width 0.25) (layer F.Cu) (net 12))
 (segment (start 161.845 115.57) (end 159.004 115.57) (width 0.25) (layer B.Cu) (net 13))
 (segment (start 159.004 115.57) (end 157.274 113.84) (width 0.25) (layer B.Cu) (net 13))
 (segment (start 157.274 113.84) (end 153.384 113.84) (width 0.25) (layer B.Cu) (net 13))
 (segment (start 158.035 107.95) (end 155.194 107.95) (width 0.25) (layer B.Cu) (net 14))
 (segment (start 155.194 107.95) (end 153.384 109.76) (width 0.25) (layer B.Cu) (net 14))
 (segment (start 153.384 109.76) (end 153.384 111.84) (width 0.25) (layer B.Cu) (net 14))
 (segment (start 160.147 111.76) (end 156.718 111.76) (width 0.25) (layer B.Cu) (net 18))
 (segment (start 156.718 111.76) (end 156.464 111.506) (width 0.25) (layer F.Cu) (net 18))
 (segment (start 156.464 111.506) (end 156.464 110.426) (width 0.25) (layer F.Cu) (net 18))
 (segment (start 156.464 110.426) (end 155.258 109.22) (width 0.25) (layer F.Cu) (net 18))
 (segment (start 155.258 109.22) (end 144.145 109.22) (width 0.25) (layer F.Cu) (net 18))
 (segment (start 144.145 109.22) (end 142.494 109.22) (width 0.25) (layer B.Cu) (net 18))
 (segment (start 167.845 111.76) (end 160.147 111.76) (width 0.25) (layer F.Cu) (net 18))
 (via (at 160.147 111.76) (size 0.6) (layers F.Cu B.Cu) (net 18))
 (via (at 156.718 111.76) (size 0.6) (layers F.Cu B.Cu) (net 18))
 (via (at 144.145 109.22) (size 0.6) (layers F.Cu B.Cu) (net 18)))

